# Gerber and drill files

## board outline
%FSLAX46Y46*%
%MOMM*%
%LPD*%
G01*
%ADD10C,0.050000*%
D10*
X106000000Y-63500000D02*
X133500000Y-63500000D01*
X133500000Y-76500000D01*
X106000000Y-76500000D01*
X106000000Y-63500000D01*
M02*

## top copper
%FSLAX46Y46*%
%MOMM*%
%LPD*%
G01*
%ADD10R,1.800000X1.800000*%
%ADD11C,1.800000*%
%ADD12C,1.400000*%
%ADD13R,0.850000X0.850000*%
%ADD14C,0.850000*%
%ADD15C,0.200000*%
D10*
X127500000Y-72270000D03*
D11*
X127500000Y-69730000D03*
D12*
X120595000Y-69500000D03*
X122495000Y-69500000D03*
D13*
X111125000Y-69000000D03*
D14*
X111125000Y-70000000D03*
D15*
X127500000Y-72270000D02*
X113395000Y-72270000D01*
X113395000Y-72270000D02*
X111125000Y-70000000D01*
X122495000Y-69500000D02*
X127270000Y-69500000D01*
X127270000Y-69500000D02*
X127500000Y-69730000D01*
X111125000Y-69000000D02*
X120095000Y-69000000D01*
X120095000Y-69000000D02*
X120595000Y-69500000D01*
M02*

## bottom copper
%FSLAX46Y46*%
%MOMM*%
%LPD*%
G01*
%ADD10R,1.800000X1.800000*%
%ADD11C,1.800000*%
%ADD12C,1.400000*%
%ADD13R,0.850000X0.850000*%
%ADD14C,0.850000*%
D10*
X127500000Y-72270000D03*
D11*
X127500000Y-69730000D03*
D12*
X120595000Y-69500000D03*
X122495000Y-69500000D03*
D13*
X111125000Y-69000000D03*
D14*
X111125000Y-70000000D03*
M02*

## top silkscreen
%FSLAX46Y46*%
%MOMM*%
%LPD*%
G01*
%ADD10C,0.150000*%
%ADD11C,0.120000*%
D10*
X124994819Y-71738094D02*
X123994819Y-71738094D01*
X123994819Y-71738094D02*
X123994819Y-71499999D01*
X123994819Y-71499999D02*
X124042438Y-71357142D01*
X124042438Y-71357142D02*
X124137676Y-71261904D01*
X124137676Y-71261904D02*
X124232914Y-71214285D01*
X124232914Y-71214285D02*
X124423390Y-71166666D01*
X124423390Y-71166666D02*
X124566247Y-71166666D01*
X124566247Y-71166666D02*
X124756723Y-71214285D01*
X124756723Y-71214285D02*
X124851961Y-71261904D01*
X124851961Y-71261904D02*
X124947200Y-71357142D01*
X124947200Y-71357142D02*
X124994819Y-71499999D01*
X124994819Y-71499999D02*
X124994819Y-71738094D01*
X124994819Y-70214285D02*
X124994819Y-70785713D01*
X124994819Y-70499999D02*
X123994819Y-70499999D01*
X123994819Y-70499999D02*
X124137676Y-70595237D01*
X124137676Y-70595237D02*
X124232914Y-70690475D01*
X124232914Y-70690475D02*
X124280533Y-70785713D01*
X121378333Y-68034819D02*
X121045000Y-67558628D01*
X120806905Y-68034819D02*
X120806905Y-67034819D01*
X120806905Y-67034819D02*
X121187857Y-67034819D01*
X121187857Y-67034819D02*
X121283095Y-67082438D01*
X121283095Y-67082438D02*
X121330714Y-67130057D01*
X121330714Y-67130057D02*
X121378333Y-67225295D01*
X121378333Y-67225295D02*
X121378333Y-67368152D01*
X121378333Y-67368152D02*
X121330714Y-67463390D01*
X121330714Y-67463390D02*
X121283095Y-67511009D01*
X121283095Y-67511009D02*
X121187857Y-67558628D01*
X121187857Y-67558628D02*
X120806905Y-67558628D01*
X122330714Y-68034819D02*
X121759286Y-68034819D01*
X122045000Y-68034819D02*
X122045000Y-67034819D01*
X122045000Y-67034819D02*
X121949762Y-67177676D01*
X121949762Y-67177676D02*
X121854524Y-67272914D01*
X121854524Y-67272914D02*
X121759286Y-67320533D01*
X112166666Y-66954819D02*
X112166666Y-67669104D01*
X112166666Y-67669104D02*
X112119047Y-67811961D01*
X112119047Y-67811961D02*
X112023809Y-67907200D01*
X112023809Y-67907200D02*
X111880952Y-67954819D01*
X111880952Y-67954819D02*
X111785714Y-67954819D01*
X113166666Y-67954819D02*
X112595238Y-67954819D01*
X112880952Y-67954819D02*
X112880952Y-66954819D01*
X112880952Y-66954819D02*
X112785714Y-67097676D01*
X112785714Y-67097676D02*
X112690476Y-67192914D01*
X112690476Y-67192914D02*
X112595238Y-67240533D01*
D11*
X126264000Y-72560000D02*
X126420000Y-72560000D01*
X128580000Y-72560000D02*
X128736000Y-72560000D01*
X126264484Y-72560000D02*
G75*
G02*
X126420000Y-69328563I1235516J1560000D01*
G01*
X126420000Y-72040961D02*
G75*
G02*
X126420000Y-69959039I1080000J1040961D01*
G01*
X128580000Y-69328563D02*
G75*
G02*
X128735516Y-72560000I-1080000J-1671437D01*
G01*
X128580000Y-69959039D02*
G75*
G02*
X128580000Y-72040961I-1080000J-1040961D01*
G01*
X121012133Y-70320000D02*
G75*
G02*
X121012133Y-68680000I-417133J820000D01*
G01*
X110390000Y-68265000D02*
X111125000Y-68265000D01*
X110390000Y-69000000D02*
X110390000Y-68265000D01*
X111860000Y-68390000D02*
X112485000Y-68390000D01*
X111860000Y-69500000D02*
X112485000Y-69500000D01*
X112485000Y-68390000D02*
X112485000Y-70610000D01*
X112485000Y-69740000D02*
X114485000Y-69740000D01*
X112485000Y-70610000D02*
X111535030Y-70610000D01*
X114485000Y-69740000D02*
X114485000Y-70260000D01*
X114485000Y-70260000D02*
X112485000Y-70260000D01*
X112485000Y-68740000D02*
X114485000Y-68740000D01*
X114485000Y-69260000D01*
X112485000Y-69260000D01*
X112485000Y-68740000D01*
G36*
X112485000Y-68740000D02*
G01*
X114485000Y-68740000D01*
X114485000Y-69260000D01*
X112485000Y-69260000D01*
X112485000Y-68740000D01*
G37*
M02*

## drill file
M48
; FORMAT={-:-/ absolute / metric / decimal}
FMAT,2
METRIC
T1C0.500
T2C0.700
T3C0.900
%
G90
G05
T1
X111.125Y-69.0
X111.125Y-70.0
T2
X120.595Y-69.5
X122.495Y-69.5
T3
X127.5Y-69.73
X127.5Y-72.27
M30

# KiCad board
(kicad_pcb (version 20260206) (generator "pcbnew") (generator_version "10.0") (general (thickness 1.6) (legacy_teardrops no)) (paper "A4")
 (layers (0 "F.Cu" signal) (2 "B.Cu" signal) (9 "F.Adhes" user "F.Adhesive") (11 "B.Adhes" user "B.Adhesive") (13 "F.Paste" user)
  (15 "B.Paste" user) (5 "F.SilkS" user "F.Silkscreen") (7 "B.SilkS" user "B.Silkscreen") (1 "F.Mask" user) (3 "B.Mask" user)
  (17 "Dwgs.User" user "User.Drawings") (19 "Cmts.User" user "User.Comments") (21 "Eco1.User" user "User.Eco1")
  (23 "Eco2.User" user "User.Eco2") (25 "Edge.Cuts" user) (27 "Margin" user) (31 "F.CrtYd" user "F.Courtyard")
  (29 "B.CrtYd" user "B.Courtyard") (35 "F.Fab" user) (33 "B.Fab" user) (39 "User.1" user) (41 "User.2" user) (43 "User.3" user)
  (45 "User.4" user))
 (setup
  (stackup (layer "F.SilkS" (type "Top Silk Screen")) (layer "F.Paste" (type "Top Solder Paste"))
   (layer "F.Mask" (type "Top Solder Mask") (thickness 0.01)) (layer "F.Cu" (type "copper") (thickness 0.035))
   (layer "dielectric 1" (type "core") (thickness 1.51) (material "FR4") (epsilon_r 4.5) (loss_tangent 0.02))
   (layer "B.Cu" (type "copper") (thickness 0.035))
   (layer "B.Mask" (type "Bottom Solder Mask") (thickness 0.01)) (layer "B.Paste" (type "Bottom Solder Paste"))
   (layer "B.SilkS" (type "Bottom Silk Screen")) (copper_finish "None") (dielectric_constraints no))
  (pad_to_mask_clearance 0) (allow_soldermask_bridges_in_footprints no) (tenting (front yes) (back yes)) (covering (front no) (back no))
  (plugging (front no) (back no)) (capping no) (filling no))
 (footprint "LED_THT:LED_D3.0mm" (layer "F.Cu") (at 127.5 72.27 90)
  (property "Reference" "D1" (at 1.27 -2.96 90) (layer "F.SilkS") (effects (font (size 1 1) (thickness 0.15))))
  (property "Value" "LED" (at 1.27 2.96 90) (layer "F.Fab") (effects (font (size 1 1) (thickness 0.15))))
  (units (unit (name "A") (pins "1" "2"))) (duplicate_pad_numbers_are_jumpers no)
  (fp_line (start -0.29 -1.236) (end -0.29 -1.08) (stroke (width 0.12) (type solid)) (layer "F.SilkS"))
  (fp_line (start -0.29 1.08) (end -0.29 1.236) (stroke (width 0.12) (type solid)) (layer "F.SilkS"))
  (fp_arc (start -0.29 -1.235516) (mid 1.36566 -1.987699) (end 2.941437 -1.08) (stroke (width 0.12) (type solid)) (layer "F.SilkS"))
  (fp_arc (start 0.229039 -1.08) (mid 1.27 -1.5) (end 2.310961 -1.08) (stroke (width 0.12) (type solid)) (layer "F.SilkS"))
  (fp_arc (start 2.941437 1.08) (mid 1.36566 1.987699) (end -0.29 1.235516) (stroke (width 0.12) (type solid)) (layer "F.SilkS"))
  (fp_arc (start 2.310961 1.08) (mid 1.27 1.5) (end 0.229039 1.08) (stroke (width 0.12) (type solid)) (layer "F.SilkS"))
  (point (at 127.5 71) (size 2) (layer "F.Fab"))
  (pad "1" thru_hole rect (at 0 0 90) (size 1.8 1.8) (drill 0.9) (layers "*.Cu" "*.Mask") (remove_unused_layers no) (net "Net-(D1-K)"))
  (pad "2" thru_hole circle (at 2.54 0 90) (size 1.8 1.8) (drill 0.9) (layers "*.Cu" "*.Mask") (remove_unused_layers no) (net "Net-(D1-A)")))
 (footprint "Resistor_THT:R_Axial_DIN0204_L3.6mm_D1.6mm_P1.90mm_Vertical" (layer "F.Cu") (at 120.595 69.5)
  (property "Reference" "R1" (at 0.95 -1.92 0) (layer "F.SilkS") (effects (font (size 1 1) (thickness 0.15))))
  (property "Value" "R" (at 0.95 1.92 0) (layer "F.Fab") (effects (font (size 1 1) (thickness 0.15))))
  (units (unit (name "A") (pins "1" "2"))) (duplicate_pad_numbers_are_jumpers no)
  (fp_arc (start 0.417133 0.82) (mid -0.92 0) (end 0.417133 -0.82) (stroke (width 0.12) (type solid)) (layer "F.SilkS"))
  (pad "1" thru_hole circle (at 0 0) (size 1.4 1.4) (drill 0.7) (layers "*.Cu" "*.Mask") (remove_unused_layers no) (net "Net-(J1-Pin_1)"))
  (pad "2" thru_hole circle (at 1.9 0) (size 1.4 1.4) (drill 0.7) (layers "*.Cu" "*.Mask") (remove_unused_layers no) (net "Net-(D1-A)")))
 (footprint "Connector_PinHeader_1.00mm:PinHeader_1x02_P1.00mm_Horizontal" (layer "F.Cu") (at 111.125 69)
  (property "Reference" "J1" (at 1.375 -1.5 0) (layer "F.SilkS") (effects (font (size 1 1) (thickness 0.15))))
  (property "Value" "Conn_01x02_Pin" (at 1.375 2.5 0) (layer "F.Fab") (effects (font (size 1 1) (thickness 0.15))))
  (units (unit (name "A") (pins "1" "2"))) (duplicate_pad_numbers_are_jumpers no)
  (fp_line (start -0.735 -0.735) (end 0 -0.735) (stroke (width 0.12) (type solid)) (layer "F.SilkS"))
  (fp_line (start -0.735 0) (end -0.735 -0.735) (stroke (width 0.12) (type solid)) (layer "F.SilkS"))
  (fp_line (start 0.735 -0.61) (end 1.36 -0.61) (stroke (width 0.12) (type solid)) (layer "F.SilkS"))
  (fp_line (start 0.735 0.5) (end 1.36 0.5) (stroke (width 0.12) (type solid)) (layer "F.SilkS"))
  (fp_line (start 1.36 -0.61) (end 1.36 1.61) (stroke (width 0.12) (type solid)) (layer "F.SilkS"))
  (fp_line (start 1.36 0.74) (end 3.36 0.74) (stroke (width 0.12) (type solid)) (layer "F.SilkS"))
  (fp_line (start 1.36 1.61) (end 0.41003 1.61) (stroke (width 0.12) (type solid)) (layer "F.SilkS"))
  (fp_line (start 3.36 0.74) (end 3.36 1.26) (stroke (width 0.12) (type solid)) (layer "F.SilkS"))
  (fp_line (start 3.36 1.26) (end 1.36 1.26) (stroke (width 0.12) (type solid)) (layer "F.SilkS"))
  (fp_rect (start 1.36 -0.26) (end 3.36 0.26) (stroke (width 0.12) (type solid)) (fill yes) (layer "F.SilkS"))
  (pad "1" thru_hole rect (at 0 0) (size 0.85 0.85) (drill 0.5) (layers "*.Cu" "*.Mask") (remove_unused_layers no) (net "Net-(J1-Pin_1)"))
  (pad "2" thru_hole circle (at 0 1) (size 0.85 0.85) (drill 0.5) (layers "*.Cu" "*.Mask") (remove_unused_layers no) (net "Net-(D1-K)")))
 (gr_rect (start 106 63.5) (end 133.5 76.5) (stroke (width 0.05) (type default)) (fill no) (layer "Edge.Cuts"))
 (segment (start 127.5 72.27) (end 113.395 72.27) (width 0.2) (layer "F.Cu") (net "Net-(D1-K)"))
 (segment (start 113.395 72.27) (end 111.125 70) (width 0.2) (layer "F.Cu") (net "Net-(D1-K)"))
 (segment (start 122.495 69.5) (end 127.27 69.5) (width 0.2) (layer "F.Cu") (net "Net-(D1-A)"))
 (segment (start 127.27 69.5) (end 127.5 69.73) (width 0.2) (layer "F.Cu") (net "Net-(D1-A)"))
 (segment (start 111.125 69) (end 120.095 69) (width 0.2) (layer "F.Cu") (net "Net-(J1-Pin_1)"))
 (segment (start 120.095 69) (end 120.595 69.5) (width 0.2) (layer "F.Cu") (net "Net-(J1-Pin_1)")))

